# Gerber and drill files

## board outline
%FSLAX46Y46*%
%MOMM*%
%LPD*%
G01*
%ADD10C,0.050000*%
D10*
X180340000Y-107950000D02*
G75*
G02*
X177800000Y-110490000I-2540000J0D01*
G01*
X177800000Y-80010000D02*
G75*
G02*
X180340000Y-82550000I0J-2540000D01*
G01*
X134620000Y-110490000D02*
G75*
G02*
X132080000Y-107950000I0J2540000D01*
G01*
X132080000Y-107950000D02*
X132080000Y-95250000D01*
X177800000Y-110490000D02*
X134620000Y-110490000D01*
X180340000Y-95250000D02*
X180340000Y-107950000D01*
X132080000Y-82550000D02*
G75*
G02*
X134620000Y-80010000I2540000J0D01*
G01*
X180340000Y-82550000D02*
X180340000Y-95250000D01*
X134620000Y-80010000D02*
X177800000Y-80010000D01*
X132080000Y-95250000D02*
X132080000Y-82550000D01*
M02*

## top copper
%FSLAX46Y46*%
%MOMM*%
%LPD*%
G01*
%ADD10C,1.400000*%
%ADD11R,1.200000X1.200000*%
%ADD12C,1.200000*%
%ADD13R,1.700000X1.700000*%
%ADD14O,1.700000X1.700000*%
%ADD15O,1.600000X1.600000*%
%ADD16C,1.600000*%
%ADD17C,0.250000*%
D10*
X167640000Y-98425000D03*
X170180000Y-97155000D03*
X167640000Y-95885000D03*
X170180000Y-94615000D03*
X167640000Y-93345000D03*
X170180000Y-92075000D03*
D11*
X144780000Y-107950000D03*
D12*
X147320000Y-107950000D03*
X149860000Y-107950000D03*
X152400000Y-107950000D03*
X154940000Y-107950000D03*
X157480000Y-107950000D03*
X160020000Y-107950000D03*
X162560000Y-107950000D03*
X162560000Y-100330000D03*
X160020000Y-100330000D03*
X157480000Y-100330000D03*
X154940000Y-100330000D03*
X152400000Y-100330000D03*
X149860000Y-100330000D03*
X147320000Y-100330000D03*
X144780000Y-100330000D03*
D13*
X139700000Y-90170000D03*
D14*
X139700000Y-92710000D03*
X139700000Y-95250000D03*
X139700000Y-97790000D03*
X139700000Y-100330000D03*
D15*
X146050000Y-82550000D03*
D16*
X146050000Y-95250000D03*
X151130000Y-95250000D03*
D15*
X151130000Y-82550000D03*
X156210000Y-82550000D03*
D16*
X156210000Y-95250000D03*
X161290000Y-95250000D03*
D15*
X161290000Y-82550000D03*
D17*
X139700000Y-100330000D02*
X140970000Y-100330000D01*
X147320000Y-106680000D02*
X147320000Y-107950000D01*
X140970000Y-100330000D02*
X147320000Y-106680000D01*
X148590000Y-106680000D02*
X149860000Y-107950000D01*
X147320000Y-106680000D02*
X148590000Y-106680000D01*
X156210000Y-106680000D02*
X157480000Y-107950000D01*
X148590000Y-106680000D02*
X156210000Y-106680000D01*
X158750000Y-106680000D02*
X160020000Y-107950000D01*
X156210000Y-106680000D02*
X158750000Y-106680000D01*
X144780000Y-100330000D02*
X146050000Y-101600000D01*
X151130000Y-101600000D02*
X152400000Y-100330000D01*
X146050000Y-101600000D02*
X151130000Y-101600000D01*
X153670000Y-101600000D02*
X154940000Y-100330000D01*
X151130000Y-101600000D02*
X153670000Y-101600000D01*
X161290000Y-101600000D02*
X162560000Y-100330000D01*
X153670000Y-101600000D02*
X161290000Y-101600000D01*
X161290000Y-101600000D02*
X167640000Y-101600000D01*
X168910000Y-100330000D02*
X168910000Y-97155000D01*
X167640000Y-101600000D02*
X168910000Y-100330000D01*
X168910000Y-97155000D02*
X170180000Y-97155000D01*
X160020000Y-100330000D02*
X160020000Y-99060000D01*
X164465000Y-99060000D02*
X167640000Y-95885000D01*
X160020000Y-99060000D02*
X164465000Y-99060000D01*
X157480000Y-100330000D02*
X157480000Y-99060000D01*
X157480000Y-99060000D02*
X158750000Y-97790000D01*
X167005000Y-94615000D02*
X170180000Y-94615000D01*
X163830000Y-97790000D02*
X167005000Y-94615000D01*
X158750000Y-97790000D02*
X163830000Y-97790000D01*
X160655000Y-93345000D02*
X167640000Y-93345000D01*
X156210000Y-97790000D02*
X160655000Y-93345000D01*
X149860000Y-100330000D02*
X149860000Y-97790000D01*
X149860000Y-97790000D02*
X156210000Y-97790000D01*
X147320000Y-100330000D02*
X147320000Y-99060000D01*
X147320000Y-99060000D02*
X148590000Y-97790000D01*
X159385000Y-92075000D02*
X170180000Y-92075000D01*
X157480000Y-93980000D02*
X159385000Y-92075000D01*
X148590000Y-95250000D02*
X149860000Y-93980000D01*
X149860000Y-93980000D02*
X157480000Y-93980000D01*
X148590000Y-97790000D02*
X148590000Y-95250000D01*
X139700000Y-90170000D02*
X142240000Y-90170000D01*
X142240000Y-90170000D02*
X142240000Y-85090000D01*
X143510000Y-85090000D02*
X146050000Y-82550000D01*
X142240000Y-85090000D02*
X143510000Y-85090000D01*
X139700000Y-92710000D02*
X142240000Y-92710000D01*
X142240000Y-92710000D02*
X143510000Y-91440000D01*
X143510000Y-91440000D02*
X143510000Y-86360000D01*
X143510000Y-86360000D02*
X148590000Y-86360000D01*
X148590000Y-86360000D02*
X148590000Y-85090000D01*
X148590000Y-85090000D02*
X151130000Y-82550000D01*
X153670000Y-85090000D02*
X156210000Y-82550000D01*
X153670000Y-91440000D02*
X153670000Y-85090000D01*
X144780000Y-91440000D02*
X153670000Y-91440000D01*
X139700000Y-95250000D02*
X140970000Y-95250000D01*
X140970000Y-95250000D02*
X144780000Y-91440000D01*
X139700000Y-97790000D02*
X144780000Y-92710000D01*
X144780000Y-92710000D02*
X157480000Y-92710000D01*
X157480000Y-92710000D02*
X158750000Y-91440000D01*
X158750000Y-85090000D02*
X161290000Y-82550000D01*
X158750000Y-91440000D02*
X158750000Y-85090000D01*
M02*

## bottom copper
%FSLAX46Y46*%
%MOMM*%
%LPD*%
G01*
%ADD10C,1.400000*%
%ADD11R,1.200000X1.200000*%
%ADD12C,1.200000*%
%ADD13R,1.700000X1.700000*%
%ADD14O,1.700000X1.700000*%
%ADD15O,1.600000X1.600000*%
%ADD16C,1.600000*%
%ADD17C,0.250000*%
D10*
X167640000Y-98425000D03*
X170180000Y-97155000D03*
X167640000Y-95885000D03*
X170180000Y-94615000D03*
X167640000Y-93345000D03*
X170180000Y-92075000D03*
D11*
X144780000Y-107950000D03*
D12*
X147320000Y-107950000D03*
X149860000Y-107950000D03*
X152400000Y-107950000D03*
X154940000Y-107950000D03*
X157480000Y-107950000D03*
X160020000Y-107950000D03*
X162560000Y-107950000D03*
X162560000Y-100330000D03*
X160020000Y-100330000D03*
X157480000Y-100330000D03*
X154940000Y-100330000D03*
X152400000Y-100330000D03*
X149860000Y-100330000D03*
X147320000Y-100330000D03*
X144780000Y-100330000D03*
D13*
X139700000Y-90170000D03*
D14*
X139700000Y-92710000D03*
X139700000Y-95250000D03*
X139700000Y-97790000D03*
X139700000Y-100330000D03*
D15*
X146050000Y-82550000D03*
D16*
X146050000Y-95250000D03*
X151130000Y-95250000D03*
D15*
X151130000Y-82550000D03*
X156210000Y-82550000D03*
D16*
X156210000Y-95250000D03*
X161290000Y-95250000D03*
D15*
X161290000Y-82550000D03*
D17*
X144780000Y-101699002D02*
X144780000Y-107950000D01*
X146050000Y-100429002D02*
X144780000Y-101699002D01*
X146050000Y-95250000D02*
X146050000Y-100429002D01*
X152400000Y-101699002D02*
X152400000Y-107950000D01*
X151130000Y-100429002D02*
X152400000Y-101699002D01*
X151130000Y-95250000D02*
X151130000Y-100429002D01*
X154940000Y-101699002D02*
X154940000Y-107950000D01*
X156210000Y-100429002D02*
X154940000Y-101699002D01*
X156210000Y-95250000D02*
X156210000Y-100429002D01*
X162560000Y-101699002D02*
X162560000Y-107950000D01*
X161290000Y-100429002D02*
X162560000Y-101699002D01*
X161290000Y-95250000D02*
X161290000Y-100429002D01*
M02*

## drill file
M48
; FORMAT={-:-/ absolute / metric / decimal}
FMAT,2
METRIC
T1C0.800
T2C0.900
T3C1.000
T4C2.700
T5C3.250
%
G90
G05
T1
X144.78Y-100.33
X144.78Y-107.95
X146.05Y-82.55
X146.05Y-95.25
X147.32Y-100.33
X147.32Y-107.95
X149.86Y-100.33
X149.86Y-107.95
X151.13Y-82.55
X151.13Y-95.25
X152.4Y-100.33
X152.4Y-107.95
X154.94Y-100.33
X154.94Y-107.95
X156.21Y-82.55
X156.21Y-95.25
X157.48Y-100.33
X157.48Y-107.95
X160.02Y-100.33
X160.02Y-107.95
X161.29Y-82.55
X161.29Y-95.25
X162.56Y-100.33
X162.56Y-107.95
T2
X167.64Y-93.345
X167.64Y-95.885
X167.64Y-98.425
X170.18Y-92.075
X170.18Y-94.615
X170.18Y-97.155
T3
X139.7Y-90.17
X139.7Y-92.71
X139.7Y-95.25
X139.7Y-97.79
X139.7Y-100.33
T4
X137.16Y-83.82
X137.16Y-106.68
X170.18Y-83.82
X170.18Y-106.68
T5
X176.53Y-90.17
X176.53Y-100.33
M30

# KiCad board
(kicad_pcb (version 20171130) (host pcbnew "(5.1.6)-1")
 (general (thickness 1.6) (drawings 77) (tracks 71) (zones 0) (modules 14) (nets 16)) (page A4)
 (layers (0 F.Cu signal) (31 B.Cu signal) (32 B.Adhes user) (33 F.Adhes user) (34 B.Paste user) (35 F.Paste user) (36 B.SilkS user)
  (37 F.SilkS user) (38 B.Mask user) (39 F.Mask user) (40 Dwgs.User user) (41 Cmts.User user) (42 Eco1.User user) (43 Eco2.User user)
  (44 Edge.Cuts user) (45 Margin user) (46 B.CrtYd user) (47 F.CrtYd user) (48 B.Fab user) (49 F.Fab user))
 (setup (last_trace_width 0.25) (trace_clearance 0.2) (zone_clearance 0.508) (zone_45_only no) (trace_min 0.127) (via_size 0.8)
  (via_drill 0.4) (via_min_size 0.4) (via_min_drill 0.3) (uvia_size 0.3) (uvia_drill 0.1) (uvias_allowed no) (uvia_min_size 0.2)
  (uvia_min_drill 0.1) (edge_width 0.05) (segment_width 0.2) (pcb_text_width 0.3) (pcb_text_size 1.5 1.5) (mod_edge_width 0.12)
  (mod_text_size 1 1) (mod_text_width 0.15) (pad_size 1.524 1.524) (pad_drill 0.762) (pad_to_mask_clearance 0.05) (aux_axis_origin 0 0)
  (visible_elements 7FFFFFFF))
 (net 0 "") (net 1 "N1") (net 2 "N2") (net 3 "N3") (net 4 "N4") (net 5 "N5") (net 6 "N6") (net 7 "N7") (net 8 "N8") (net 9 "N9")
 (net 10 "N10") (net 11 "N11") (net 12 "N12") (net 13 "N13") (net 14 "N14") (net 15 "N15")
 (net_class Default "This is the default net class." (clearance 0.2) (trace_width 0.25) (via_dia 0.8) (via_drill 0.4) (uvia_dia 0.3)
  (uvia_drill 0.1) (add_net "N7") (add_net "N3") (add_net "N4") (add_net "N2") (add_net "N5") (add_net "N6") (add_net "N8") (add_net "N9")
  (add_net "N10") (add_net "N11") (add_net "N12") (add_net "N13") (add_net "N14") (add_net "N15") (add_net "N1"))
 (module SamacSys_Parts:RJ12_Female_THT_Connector (layer F.Cu) (at 176.53 90.17 90)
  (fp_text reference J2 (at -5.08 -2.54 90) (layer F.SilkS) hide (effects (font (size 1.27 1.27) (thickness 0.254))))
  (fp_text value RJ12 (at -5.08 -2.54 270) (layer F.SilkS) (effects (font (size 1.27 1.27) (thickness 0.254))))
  (pad 1 thru_hole circle (at -8.255 -8.89 90) (size 1.4 1.4) (drill 0.9) (layers *.Cu *.Mask) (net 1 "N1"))
  (pad 2 thru_hole circle (at -6.985 -6.35 90) (size 1.4 1.4) (drill 0.9) (layers *.Cu *.Mask) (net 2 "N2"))
  (pad 3 thru_hole circle (at -5.715 -8.89 90) (size 1.4 1.4) (drill 0.9) (layers *.Cu *.Mask) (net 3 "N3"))
  (pad 4 thru_hole circle (at -4.445 -6.35 90) (size 1.4 1.4) (drill 0.9) (layers *.Cu *.Mask) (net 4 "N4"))
  (pad 5 thru_hole circle (at -3.175 -8.89 90) (size 1.4 1.4) (drill 0.9) (layers *.Cu *.Mask) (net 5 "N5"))
  (pad 6 thru_hole circle (at -1.905 -6.35 90) (size 1.4 1.4) (drill 0.9) (layers *.Cu *.Mask) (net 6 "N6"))
  (pad 7 np_thru_hole circle (at -10.16 0 90) (size 3.25 0) (drill 3.25) (layers *.Cu *.Mask))
  (pad 8 np_thru_hole circle (at 0 0 90) (size 3.25 0) (drill 3.25) (layers *.Cu *.Mask)))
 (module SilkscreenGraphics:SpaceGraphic (layer B.Cu) (at 148.59 88.9 180)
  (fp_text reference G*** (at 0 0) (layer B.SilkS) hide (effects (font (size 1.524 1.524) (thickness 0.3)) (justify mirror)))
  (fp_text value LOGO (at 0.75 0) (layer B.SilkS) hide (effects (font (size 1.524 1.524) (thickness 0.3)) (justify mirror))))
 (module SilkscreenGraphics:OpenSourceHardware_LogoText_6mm (layer B.Cu) (at 158.75 88.9 180)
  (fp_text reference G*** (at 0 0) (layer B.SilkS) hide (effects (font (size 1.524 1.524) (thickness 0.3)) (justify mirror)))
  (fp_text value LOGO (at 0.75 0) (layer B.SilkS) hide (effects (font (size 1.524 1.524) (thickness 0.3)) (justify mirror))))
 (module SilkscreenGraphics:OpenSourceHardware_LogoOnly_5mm (layer F.Cu) (at 176.53 83.82)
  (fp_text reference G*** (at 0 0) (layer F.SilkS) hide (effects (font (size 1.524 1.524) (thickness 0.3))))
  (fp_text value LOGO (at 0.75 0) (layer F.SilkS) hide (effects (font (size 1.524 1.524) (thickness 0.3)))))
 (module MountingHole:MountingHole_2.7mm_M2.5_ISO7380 (layer F.Cu) (at 137.16 83.82)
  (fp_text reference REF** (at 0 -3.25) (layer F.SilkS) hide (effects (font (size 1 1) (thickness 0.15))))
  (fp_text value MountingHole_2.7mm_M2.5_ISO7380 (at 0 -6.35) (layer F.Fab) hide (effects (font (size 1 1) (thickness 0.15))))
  (pad 1 np_thru_hole circle (at 0 0) (size 2.7 2.7) (drill 2.7) (layers *.Cu *.Mask)))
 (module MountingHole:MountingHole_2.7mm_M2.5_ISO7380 (layer F.Cu) (at 137.16 106.68)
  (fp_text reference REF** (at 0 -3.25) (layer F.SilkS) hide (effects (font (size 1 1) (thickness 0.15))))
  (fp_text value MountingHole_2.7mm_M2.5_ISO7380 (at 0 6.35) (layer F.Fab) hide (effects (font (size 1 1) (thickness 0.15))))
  (pad 1 np_thru_hole circle (at 0 0) (size 2.7 2.7) (drill 2.7) (layers *.Cu *.Mask)))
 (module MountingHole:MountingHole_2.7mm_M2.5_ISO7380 (layer F.Cu) (at 170.18 106.68)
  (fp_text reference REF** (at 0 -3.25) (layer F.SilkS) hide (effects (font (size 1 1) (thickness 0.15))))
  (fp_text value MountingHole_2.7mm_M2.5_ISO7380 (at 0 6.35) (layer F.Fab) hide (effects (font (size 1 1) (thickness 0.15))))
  (pad 1 np_thru_hole circle (at 0 0) (size 2.7 2.7) (drill 2.7) (layers *.Cu *.Mask)))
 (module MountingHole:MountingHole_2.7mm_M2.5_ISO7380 (layer F.Cu) (at 170.18 83.82)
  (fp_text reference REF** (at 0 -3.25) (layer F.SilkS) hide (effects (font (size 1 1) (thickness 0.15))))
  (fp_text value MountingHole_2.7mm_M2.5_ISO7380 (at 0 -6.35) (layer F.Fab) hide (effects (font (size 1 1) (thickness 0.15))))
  (pad 1 np_thru_hole circle (at 0 0) (size 2.7 2.7) (drill 2.7) (layers *.Cu *.Mask)))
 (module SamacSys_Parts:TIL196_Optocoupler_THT (layer F.Cu) (at 153.67 104.14 90)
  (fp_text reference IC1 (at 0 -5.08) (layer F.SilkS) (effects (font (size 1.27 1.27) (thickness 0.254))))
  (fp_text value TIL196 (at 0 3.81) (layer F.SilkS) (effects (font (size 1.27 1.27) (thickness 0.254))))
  (pad 1 thru_hole rect (at -3.81 -8.89 90) (size 1.2 1.2) (drill 0.8) (layers *.Cu *.Mask) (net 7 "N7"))
  (pad 2 thru_hole circle (at -3.81 -6.35 90) (size 1.2 1.2) (drill 0.8) (layers *.Cu *.Mask) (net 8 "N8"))
  (pad 3 thru_hole circle (at -3.81 -3.81 90) (size 1.2 1.2) (drill 0.8) (layers *.Cu *.Mask) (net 8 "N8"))
  (pad 4 thru_hole circle (at -3.81 -1.27 90) (size 1.2 1.2) (drill 0.8) (layers *.Cu *.Mask) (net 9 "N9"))
  (pad 5 thru_hole circle (at -3.81 1.27 90) (size 1.2 1.2) (drill 0.8) (layers *.Cu *.Mask) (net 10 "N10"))
  (pad 6 thru_hole circle (at -3.81 3.81 90) (size 1.2 1.2) (drill 0.8) (layers *.Cu *.Mask) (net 8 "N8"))
  (pad 7 thru_hole circle (at -3.81 6.35 90) (size 1.2 1.2) (drill 0.8) (layers *.Cu *.Mask) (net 8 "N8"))
  (pad 8 thru_hole circle (at -3.81 8.89 90) (size 1.2 1.2) (drill 0.8) (layers *.Cu *.Mask) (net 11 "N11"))
  (pad 9 thru_hole circle (at 3.81 8.89 90) (size 1.2 1.2) (drill 0.8) (layers *.Cu *.Mask) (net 2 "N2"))
  (pad 10 thru_hole circle (at 3.81 6.35 90) (size 1.2 1.2) (drill 0.8) (layers *.Cu *.Mask) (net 3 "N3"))
  (pad 11 thru_hole circle (at 3.81 3.81 90) (size 1.2 1.2) (drill 0.8) (layers *.Cu *.Mask) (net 4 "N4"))
  (pad 12 thru_hole circle (at 3.81 1.27 90) (size 1.2 1.2) (drill 0.8) (layers *.Cu *.Mask) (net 2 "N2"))
  (pad 13 thru_hole circle (at 3.81 -1.27 90) (size 1.2 1.2) (drill 0.8) (layers *.Cu *.Mask) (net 2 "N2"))
  (pad 14 thru_hole circle (at 3.81 -3.81 90) (size 1.2 1.2) (drill 0.8) (layers *.Cu *.Mask) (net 5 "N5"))
  (pad 15 thru_hole circle (at 3.81 -6.35 90) (size 1.2 1.2) (drill 0.8) (layers *.Cu *.Mask) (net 6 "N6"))
  (pad 16 thru_hole circle (at 3.81 -8.89 90) (size 1.2 1.2) (drill 0.8) (layers *.Cu *.Mask) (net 2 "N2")))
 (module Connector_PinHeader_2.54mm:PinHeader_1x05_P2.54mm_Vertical (layer F.Cu) (at 139.7 90.17)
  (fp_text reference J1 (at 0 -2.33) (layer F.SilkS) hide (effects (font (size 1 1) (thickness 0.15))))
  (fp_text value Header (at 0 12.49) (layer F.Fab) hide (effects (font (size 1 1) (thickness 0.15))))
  (pad 1 thru_hole rect (at 0 0) (size 1.7 1.7) (drill 1) (layers *.Cu *.Mask) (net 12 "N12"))
  (pad 2 thru_hole oval (at 0 2.54) (size 1.7 1.7) (drill 1) (layers *.Cu *.Mask) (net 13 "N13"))
  (pad 3 thru_hole oval (at 0 5.08) (size 1.7 1.7) (drill 1) (layers *.Cu *.Mask) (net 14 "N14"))
  (pad 4 thru_hole oval (at 0 7.62) (size 1.7 1.7) (drill 1) (layers *.Cu *.Mask) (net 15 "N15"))
  (pad 5 thru_hole oval (at 0 10.16) (size 1.7 1.7) (drill 1) (layers *.Cu *.Mask) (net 8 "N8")))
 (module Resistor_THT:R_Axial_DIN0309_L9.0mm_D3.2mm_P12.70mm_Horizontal (layer F.Cu) (at 146.05 95.25 90)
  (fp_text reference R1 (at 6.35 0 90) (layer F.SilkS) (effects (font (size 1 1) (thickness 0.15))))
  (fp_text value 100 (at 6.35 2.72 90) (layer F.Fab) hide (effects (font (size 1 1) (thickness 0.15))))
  (pad 2 thru_hole oval (at 12.7 0 90) (size 1.6 1.6) (drill 0.8) (layers *.Cu *.Mask) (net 12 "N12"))
  (pad 1 thru_hole circle (at 0 0 90) (size 1.6 1.6) (drill 0.8) (layers *.Cu *.Mask) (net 7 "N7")))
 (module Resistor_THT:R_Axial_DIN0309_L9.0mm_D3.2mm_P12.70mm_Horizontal (layer F.Cu) (at 151.13 95.25 90)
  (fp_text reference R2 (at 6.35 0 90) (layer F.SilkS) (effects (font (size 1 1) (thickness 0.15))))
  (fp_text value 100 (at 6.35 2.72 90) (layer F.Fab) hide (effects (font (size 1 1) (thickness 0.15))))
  (pad 1 thru_hole circle (at 0 0 90) (size 1.6 1.6) (drill 0.8) (layers *.Cu *.Mask) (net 9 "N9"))
  (pad 2 thru_hole oval (at 12.7 0 90) (size 1.6 1.6) (drill 0.8) (layers *.Cu *.Mask) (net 13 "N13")))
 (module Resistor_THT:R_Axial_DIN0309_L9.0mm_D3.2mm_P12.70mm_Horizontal (layer F.Cu) (at 156.21 95.25 90)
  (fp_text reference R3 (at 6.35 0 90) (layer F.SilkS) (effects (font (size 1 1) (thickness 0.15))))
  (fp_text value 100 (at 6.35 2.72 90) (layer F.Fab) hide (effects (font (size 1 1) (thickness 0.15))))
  (pad 2 thru_hole oval (at 12.7 0 90) (size 1.6 1.6) (drill 0.8) (layers *.Cu *.Mask) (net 14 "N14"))
  (pad 1 thru_hole circle (at 0 0 90) (size 1.6 1.6) (drill 0.8) (layers *.Cu *.Mask) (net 10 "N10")))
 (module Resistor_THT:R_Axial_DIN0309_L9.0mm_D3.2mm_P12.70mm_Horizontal (layer F.Cu) (at 161.29 95.25 90)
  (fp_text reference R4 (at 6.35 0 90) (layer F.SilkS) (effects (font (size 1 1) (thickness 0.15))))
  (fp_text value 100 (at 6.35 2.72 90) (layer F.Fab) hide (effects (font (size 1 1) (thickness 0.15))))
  (pad 1 thru_hole circle (at 0 0 90) (size 1.6 1.6) (drill 0.8) (layers *.Cu *.Mask) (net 11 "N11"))
  (pad 2 thru_hole oval (at 12.7 0 90) (size 1.6 1.6) (drill 0.8) (layers *.Cu *.Mask) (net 15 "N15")))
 (gr_arc (start 177.8 107.95) (end 177.8 110.49) (angle -90) (layer Edge.Cuts) (width 0.05))
 (gr_arc (start 177.8 82.55) (end 180.34 82.55) (angle -90) (layer Edge.Cuts) (width 0.05))
 (gr_arc (start 134.62 107.95) (end 132.08 107.95) (angle -90) (layer Edge.Cuts) (width 0.05))
 (gr_line (start 132.08 107.95) (end 132.08 95.25) (layer Edge.Cuts) (width 0.05))
 (gr_line (start 177.8 110.49) (end 134.62 110.49) (layer Edge.Cuts) (width 0.05))
 (gr_line (start 180.34 95.25) (end 180.34 107.95) (layer Edge.Cuts) (width 0.05))
 (gr_arc (start 134.62 82.55) (end 134.62 80.01) (angle -90) (layer Edge.Cuts) (width 0.05))
 (gr_line (start 180.34 82.55) (end 180.34 95.25) (layer Edge.Cuts) (width 0.05))
 (gr_line (start 134.62 80.01) (end 177.8 80.01) (layer Edge.Cuts) (width 0.05))
 (gr_line (start 132.08 95.25) (end 132.08 82.55) (layer Edge.Cuts) (width 0.05))
 (segment (start 144.78 101.699002) (end 144.78 107.95) (width 0.25) (layer B.Cu) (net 7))
 (segment (start 146.05 100.429002) (end 144.78 101.699002) (width 0.25) (layer B.Cu) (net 7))
 (segment (start 146.05 95.25) (end 146.05 100.429002) (width 0.25) (layer B.Cu) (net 7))
 (segment (start 139.7 100.33) (end 140.97 100.33) (width 0.25) (layer F.Cu) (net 8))
 (segment (start 147.32 106.68) (end 147.32 107.95) (width 0.25) (layer F.Cu) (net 8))
 (segment (start 140.97 100.33) (end 147.32 106.68) (width 0.25) (layer F.Cu) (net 8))
 (segment (start 148.59 106.68) (end 149.86 107.95) (width 0.25) (layer F.Cu) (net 8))
 (segment (start 147.32 106.68) (end 148.59 106.68) (width 0.25) (layer F.Cu) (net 8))
 (segment (start 156.21 106.68) (end 157.48 107.95) (width 0.25) (layer F.Cu) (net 8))
 (segment (start 148.59 106.68) (end 156.21 106.68) (width 0.25) (layer F.Cu) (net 8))
 (segment (start 158.75 106.68) (end 160.02 107.95) (width 0.25) (layer F.Cu) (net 8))
 (segment (start 156.21 106.68) (end 158.75 106.68) (width 0.25) (layer F.Cu) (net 8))
 (segment (start 152.4 101.699002) (end 152.4 107.95) (width 0.25) (layer B.Cu) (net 9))
 (segment (start 151.13 100.429002) (end 152.4 101.699002) (width 0.25) (layer B.Cu) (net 9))
 (segment (start 151.13 95.25) (end 151.13 100.429002) (width 0.25) (layer B.Cu) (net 9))
 (segment (start 154.94 101.699002) (end 154.94 107.95) (width 0.25) (layer B.Cu) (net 10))
 (segment (start 156.21 100.429002) (end 154.94 101.699002) (width 0.25) (layer B.Cu) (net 10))
 (segment (start 156.21 95.25) (end 156.21 100.429002) (width 0.25) (layer B.Cu) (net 10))
 (segment (start 162.56 101.699002) (end 162.56 107.95) (width 0.25) (layer B.Cu) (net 11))
 (segment (start 161.29 100.429002) (end 162.56 101.699002) (width 0.25) (layer B.Cu) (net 11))
 (segment (start 161.29 95.25) (end 161.29 100.429002) (width 0.25) (layer B.Cu) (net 11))
 (segment (start 144.78 100.33) (end 146.05 101.6) (width 0.25) (layer F.Cu) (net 2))
 (segment (start 151.13 101.6) (end 152.4 100.33) (width 0.25) (layer F.Cu) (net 2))
 (segment (start 146.05 101.6) (end 151.13 101.6) (width 0.25) (layer F.Cu) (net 2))
 (segment (start 153.67 101.6) (end 154.94 100.33) (width 0.25) (layer F.Cu) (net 2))
 (segment (start 151.13 101.6) (end 153.67 101.6) (width 0.25) (layer F.Cu) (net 2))
 (segment (start 161.29 101.6) (end 162.56 100.33) (width 0.25) (layer F.Cu) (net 2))
 (segment (start 153.67 101.6) (end 161.29 101.6) (width 0.25) (layer F.Cu) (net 2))
 (segment (start 161.29 101.6) (end 167.64 101.6) (width 0.25) (layer F.Cu) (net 2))
 (segment (start 168.91 100.33) (end 168.91 97.155) (width 0.25) (layer F.Cu) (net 2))
 (segment (start 167.64 101.6) (end 168.91 100.33) (width 0.25) (layer F.Cu) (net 2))
 (segment (start 168.91 97.155) (end 170.18 97.155) (width 0.25) (layer F.Cu) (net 2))
 (segment (start 160.02 100.33) (end 160.02 99.06) (width 0.25) (layer F.Cu) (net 3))
 (segment (start 164.465 99.06) (end 167.64 95.885) (width 0.25) (layer F.Cu) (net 3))
 (segment (start 160.02 99.06) (end 164.465 99.06) (width 0.25) (layer F.Cu) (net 3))
 (segment (start 157.48 100.33) (end 157.48 99.06) (width 0.25) (layer F.Cu) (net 4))
 (segment (start 157.48 99.06) (end 158.75 97.79) (width 0.25) (layer F.Cu) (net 4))
 (segment (start 167.005 94.615) (end 170.18 94.615) (width 0.25) (layer F.Cu) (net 4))
 (segment (start 163.83 97.79) (end 167.005 94.615) (width 0.25) (layer F.Cu) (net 4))
 (segment (start 158.75 97.79) (end 163.83 97.79) (width 0.25) (layer F.Cu) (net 4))
 (segment (start 160.655 93.345) (end 167.64 93.345) (width 0.25) (layer F.Cu) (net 5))
 (segment (start 156.21 97.79) (end 160.655 93.345) (width 0.25) (layer F.Cu) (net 5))
 (segment (start 149.86 100.33) (end 149.86 97.79) (width 0.25) (layer F.Cu) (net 5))
 (segment (start 149.86 97.79) (end 156.21 97.79) (width 0.25) (layer F.Cu) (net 5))
 (segment (start 147.32 100.33) (end 147.32 99.06) (width 0.25) (layer F.Cu) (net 6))
 (segment (start 147.32 99.06) (end 148.59 97.79) (width 0.25) (layer F.Cu) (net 6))
 (segment (start 159.385 92.075) (end 170.18 92.075) (width 0.25) (layer F.Cu) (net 6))
 (segment (start 157.48 93.98) (end 159.385 92.075) (width 0.25) (layer F.Cu) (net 6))
 (segment (start 148.59 95.25) (end 149.86 93.98) (width 0.25) (layer F.Cu) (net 6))
 (segment (start 149.86 93.98) (end 157.48 93.98) (width 0.25) (layer F.Cu) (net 6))
 (segment (start 148.59 97.79) (end 148.59 95.25) (width 0.25) (layer F.Cu) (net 6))
 (segment (start 139.7 90.17) (end 142.24 90.17) (width 0.25) (layer F.Cu) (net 12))
 (segment (start 142.24 90.17) (end 142.24 85.09) (width 0.25) (layer F.Cu) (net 12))
 (segment (start 143.51 85.09) (end 146.05 82.55) (width 0.25) (layer F.Cu) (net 12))
 (segment (start 142.24 85.09) (end 143.51 85.09) (width 0.25) (layer F.Cu) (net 12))
 (segment (start 139.7 92.71) (end 142.24 92.71) (width 0.25) (layer F.Cu) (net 13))
 (segment (start 142.24 92.71) (end 143.51 91.44) (width 0.25) (layer F.Cu) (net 13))
 (segment (start 143.51 91.44) (end 143.51 86.36) (width 0.25) (layer F.Cu) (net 13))
 (segment (start 143.51 86.36) (end 148.59 86.36) (width 0.25) (layer F.Cu) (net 13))
 (segment (start 148.59 86.36) (end 148.59 85.09) (width 0.25) (layer F.Cu) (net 13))
 (segment (start 148.59 85.09) (end 151.13 82.55) (width 0.25) (layer F.Cu) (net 13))
 (segment (start 153.67 85.09) (end 156.21 82.55) (width 0.25) (layer F.Cu) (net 14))
 (segment (start 153.67 91.44) (end 153.67 85.09) (width 0.25) (layer F.Cu) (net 14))
 (segment (start 144.78 91.44) (end 153.67 91.44) (width 0.25) (layer F.Cu) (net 14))
 (segment (start 139.7 95.25) (end 140.97 95.25) (width 0.25) (layer F.Cu) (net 14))
 (segment (start 140.97 95.25) (end 144.78 91.44) (width 0.25) (layer F.Cu) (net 14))
 (segment (start 139.7 97.79) (end 144.78 92.71) (width 0.25) (layer F.Cu) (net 15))
 (segment (start 144.78 92.71) (end 157.48 92.71) (width 0.25) (layer F.Cu) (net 15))
 (segment (start 157.48 92.71) (end 158.75 91.44) (width 0.25) (layer F.Cu) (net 15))
 (segment (start 158.75 85.09) (end 161.29 82.55) (width 0.25) (layer F.Cu) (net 15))
 (segment (start 158.75 91.44) (end 158.75 85.09) (width 0.25) (layer F.Cu) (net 15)))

